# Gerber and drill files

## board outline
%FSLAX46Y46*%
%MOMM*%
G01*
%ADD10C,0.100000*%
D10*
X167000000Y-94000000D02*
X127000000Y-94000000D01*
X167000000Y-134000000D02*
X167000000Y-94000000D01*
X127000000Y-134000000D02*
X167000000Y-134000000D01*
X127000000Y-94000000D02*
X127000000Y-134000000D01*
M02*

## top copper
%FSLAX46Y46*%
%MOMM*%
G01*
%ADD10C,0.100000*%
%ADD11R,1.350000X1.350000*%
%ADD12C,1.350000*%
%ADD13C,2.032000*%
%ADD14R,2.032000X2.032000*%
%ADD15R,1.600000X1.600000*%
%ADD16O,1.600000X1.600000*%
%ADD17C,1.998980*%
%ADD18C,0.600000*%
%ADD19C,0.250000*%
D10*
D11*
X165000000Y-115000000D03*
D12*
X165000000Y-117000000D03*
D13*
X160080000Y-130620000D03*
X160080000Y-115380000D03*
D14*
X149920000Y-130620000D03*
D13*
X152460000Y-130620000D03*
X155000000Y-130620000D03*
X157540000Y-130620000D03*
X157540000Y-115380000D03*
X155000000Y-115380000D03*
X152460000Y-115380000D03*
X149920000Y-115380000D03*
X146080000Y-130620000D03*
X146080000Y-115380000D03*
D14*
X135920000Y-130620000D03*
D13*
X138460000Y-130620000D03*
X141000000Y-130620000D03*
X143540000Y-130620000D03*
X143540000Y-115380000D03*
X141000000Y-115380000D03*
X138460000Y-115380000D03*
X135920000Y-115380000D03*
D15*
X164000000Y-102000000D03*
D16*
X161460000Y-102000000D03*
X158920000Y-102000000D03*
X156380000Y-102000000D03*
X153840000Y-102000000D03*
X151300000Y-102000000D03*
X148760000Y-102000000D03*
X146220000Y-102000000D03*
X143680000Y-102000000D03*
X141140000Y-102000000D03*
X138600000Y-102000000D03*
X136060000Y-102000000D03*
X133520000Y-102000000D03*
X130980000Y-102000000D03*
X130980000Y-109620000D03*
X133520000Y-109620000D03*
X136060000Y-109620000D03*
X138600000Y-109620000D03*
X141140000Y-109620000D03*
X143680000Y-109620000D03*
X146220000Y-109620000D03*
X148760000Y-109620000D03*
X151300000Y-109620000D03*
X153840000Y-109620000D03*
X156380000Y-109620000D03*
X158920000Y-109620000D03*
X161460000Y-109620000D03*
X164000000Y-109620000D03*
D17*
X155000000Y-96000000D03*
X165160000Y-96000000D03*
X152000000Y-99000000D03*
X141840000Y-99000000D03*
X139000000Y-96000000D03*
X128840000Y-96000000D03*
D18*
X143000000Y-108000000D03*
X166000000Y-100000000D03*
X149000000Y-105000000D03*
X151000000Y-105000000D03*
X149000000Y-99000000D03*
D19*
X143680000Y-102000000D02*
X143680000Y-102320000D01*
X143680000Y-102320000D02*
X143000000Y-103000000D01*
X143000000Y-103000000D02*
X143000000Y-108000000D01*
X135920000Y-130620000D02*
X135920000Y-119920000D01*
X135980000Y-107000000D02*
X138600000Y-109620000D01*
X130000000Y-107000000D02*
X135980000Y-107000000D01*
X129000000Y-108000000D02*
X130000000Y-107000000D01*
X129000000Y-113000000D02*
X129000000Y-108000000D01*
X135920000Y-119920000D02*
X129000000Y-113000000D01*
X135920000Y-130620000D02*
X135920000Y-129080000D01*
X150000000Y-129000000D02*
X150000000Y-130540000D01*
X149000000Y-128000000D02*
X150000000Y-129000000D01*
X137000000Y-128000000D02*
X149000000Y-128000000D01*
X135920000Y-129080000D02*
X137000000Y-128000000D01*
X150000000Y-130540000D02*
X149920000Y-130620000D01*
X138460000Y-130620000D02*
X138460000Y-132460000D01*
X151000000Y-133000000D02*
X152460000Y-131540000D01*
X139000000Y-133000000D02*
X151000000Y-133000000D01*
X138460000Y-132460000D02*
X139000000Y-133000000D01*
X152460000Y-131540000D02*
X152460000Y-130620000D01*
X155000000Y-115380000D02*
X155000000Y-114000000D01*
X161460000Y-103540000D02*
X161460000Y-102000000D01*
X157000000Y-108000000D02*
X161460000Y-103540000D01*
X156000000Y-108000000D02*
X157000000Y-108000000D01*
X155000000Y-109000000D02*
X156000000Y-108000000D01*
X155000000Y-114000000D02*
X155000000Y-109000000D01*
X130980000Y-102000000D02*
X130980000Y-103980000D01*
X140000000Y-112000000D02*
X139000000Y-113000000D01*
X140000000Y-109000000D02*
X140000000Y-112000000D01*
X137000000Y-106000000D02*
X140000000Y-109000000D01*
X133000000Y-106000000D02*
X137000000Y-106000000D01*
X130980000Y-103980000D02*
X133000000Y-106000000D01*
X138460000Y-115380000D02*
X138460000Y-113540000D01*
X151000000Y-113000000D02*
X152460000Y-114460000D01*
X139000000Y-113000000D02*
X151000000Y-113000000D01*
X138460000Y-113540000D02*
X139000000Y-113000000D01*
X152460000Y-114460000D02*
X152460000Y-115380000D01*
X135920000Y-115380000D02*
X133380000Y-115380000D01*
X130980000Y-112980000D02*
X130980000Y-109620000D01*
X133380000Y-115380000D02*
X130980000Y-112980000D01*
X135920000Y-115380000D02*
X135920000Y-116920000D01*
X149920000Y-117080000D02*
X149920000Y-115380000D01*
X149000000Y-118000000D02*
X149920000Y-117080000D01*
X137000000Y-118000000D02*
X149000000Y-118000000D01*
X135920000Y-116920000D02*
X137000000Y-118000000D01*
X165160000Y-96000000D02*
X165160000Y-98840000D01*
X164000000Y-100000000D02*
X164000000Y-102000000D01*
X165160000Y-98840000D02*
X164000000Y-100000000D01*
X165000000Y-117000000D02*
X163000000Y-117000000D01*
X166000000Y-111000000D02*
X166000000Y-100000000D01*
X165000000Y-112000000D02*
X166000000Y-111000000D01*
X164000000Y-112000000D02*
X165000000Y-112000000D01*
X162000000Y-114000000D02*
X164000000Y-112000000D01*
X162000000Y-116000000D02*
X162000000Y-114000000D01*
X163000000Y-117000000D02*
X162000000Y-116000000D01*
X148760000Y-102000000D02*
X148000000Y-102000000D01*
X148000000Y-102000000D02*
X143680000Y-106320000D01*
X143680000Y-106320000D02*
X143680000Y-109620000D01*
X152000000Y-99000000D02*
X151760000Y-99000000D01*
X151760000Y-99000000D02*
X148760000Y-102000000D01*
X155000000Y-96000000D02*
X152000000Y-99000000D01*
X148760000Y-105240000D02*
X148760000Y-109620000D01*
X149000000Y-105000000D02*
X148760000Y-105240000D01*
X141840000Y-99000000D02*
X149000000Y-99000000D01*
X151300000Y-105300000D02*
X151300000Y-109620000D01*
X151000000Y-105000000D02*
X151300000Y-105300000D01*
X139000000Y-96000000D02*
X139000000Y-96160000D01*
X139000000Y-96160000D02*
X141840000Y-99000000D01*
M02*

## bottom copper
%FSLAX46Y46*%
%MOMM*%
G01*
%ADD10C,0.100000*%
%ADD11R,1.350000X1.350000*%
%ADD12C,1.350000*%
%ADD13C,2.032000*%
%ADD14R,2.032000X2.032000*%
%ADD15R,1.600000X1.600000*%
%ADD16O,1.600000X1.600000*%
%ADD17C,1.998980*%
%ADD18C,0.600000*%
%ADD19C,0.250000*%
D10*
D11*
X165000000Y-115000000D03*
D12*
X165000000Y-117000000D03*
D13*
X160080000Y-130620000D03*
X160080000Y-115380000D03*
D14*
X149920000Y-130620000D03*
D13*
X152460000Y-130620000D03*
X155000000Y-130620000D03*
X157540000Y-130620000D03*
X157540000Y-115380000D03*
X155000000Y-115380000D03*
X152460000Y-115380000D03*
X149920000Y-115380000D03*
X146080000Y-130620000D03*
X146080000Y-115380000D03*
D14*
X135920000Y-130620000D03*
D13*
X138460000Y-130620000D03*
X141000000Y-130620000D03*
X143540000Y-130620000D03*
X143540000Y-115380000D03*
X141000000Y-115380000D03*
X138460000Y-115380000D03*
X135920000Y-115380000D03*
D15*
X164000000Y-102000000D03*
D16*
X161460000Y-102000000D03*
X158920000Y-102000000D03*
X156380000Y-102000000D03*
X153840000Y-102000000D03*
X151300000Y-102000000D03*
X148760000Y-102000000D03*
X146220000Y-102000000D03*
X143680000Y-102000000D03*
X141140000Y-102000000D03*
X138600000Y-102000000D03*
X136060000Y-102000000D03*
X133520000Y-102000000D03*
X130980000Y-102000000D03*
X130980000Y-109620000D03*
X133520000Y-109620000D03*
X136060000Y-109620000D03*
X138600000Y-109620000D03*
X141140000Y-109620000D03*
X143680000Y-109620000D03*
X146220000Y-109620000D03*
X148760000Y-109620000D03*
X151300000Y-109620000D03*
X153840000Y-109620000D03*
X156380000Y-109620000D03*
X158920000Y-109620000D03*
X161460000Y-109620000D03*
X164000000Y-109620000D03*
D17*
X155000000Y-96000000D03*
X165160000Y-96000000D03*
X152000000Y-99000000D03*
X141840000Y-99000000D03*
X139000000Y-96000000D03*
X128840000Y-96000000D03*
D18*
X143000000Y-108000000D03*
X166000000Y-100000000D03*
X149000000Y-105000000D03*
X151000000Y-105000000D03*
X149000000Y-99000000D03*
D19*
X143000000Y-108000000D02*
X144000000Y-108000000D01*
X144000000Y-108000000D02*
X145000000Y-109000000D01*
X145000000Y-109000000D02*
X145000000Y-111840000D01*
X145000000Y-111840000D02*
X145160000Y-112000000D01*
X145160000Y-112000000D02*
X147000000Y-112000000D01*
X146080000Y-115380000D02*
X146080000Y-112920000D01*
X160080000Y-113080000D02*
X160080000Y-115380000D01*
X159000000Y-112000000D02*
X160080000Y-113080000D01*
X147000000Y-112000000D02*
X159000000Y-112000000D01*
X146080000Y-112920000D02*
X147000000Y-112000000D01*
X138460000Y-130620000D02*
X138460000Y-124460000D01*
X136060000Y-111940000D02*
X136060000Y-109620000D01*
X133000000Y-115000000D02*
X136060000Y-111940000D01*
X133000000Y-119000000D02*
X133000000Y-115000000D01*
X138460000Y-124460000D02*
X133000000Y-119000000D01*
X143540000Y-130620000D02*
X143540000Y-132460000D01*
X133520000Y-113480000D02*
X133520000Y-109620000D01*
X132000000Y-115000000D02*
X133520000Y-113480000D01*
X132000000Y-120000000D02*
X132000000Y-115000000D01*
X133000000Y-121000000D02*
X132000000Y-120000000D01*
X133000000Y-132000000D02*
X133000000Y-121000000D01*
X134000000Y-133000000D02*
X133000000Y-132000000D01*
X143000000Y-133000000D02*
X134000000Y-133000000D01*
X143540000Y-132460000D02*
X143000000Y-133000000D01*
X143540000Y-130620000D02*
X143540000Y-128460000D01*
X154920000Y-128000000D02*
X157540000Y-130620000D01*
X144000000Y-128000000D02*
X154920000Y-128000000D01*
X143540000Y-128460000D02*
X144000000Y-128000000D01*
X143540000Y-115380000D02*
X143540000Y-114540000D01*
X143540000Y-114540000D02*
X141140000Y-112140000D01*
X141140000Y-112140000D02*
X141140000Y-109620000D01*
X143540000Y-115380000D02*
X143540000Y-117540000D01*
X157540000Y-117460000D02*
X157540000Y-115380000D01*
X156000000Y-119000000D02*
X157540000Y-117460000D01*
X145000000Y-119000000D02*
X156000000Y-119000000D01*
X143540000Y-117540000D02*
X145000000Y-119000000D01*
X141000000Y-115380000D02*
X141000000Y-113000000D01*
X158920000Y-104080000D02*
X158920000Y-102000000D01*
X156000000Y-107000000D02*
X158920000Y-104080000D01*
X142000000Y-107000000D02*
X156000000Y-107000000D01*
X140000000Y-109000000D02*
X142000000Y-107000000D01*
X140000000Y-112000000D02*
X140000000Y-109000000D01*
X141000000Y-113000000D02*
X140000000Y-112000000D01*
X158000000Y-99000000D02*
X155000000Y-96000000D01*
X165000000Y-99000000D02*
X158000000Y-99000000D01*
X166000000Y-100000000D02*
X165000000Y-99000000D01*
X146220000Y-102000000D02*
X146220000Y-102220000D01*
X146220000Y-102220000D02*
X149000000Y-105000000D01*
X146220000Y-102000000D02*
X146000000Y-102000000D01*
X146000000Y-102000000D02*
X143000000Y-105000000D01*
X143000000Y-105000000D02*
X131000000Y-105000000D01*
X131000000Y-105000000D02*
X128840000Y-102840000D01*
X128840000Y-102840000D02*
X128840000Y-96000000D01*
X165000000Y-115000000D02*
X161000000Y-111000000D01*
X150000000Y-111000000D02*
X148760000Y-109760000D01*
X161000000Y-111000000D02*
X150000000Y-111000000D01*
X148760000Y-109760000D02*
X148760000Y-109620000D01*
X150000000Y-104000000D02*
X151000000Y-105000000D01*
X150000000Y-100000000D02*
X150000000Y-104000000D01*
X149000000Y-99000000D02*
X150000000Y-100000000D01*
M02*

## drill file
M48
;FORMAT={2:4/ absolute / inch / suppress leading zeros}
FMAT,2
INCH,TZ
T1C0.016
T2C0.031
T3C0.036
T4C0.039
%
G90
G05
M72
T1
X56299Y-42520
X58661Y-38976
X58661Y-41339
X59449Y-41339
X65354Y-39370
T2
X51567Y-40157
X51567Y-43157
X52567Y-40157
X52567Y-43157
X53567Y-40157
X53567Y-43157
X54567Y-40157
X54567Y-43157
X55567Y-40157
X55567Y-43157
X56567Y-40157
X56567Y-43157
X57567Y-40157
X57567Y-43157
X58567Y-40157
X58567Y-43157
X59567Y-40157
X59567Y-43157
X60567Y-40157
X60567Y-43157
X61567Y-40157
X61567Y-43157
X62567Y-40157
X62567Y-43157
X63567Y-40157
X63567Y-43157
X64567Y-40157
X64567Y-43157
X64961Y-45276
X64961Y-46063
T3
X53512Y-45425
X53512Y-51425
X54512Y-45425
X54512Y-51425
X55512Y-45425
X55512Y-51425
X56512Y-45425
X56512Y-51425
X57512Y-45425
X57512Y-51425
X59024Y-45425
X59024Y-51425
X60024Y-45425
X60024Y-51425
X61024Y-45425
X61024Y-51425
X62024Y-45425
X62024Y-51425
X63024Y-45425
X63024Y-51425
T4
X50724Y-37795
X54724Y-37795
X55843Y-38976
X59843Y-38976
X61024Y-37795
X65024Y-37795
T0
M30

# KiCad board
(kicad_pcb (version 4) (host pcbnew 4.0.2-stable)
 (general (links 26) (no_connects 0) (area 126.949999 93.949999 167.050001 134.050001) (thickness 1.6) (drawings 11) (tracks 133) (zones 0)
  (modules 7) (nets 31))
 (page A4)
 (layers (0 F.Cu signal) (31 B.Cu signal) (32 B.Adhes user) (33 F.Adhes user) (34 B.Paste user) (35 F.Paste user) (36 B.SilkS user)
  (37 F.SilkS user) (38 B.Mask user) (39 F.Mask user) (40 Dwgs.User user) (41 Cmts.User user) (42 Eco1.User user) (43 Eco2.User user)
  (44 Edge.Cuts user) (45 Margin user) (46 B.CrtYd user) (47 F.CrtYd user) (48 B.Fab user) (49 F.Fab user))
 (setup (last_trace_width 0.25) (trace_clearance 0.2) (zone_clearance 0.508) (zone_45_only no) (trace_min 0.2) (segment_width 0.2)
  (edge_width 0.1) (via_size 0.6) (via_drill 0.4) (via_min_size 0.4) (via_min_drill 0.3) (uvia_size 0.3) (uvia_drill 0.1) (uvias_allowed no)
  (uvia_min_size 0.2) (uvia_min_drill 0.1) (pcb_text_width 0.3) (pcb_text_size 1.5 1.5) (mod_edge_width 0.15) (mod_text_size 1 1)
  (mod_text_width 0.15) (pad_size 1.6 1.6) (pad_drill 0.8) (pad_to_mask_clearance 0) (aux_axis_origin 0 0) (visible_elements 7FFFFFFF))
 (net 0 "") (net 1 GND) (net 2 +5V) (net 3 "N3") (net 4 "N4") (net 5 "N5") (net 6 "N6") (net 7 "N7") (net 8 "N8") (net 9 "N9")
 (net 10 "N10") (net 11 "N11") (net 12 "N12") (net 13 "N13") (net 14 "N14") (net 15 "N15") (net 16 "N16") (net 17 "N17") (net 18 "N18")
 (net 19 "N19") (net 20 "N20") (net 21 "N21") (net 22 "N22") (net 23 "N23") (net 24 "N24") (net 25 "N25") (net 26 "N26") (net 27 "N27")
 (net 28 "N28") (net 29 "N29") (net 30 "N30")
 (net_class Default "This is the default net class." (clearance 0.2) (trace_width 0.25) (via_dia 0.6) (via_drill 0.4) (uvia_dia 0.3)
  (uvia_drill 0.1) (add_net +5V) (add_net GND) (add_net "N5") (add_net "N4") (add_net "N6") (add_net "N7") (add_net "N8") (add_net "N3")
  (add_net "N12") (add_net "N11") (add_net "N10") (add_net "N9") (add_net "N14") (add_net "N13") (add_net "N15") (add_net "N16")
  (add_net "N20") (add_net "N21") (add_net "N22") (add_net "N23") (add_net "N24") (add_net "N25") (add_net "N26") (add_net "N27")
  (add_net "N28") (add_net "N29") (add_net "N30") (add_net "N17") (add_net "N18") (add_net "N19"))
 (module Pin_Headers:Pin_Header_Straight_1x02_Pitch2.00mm (layer F.Cu) (at 165 115)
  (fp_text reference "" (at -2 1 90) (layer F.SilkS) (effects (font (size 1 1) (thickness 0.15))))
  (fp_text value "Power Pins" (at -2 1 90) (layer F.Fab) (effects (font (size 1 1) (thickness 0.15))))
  (pad 1 thru_hole rect (at 0 0) (size 1.35 1.35) (drill 0.8) (layers *.Cu *.Mask) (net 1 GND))
  (pad 2 thru_hole circle (at 0 2) (size 1.35 1.35) (drill 0.8) (layers *.Cu *.Mask) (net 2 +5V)))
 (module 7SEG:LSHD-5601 (layer F.Cu) (at 155 123)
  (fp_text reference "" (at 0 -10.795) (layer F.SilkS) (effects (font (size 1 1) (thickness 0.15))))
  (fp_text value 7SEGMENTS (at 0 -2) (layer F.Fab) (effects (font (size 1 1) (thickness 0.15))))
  (pad 5 thru_hole circle (at 5.08 7.62) (size 2.032 2.032) (drill 0.9144) (layers *.Cu *.Mask F.SilkS) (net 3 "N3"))
  (pad 10 thru_hole circle (at 5.08 -7.62) (size 2.032 2.032) (drill 0.9144) (layers *.Cu *.Mask F.SilkS) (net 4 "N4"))
  (pad 1 thru_hole rect (at -5.08 7.62) (size 2.032 2.032) (drill 0.9144) (layers *.Cu *.Mask F.SilkS) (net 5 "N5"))
  (pad 2 thru_hole circle (at -2.54 7.62) (size 2.032 2.032) (drill 0.9144) (layers *.Cu *.Mask F.SilkS) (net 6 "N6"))
  (pad 3 thru_hole circle (at 0 7.62) (size 2.032 2.032) (drill 0.9144) (layers *.Cu *.Mask F.SilkS) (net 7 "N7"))
  (pad 4 thru_hole circle (at 2.54 7.62) (size 2.032 2.032) (drill 0.9144) (layers *.Cu *.Mask F.SilkS) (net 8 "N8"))
  (pad 9 thru_hole circle (at 2.54 -7.62) (size 2.032 2.032) (drill 0.9144) (layers *.Cu *.Mask F.SilkS) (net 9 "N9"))
  (pad 8 thru_hole circle (at 0 -7.62) (size 2.032 2.032) (drill 0.9144) (layers *.Cu *.Mask F.SilkS) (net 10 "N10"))
  (pad 7 thru_hole circle (at -2.54 -7.62) (size 2.032 2.032) (drill 0.9144) (layers *.Cu *.Mask F.SilkS) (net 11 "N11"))
  (pad 6 thru_hole circle (at -5.08 -7.62) (size 2.032 2.032) (drill 0.9144) (layers *.Cu *.Mask F.SilkS) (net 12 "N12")))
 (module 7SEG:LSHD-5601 (layer F.Cu) (at 141 123)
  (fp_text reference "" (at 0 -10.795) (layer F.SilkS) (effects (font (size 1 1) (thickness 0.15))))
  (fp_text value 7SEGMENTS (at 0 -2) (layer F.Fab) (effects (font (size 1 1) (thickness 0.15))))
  (pad 5 thru_hole circle (at 5.08 7.62) (size 2.032 2.032) (drill 0.9144) (layers *.Cu *.Mask F.SilkS) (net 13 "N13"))
  (pad 10 thru_hole circle (at 5.08 -7.62) (size 2.032 2.032) (drill 0.9144) (layers *.Cu *.Mask F.SilkS) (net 4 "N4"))
  (pad 1 thru_hole rect (at -5.08 7.62) (size 2.032 2.032) (drill 0.9144) (layers *.Cu *.Mask F.SilkS) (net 5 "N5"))
  (pad 2 thru_hole circle (at -2.54 7.62) (size 2.032 2.032) (drill 0.9144) (layers *.Cu *.Mask F.SilkS) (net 6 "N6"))
  (pad 3 thru_hole circle (at 0 7.62) (size 2.032 2.032) (drill 0.9144) (layers *.Cu *.Mask F.SilkS) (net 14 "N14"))
  (pad 4 thru_hole circle (at 2.54 7.62) (size 2.032 2.032) (drill 0.9144) (layers *.Cu *.Mask F.SilkS) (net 8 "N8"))
  (pad 9 thru_hole circle (at 2.54 -7.62) (size 2.032 2.032) (drill 0.9144) (layers *.Cu *.Mask F.SilkS) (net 9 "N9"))
  (pad 8 thru_hole circle (at 0 -7.62) (size 2.032 2.032) (drill 0.9144) (layers *.Cu *.Mask F.SilkS) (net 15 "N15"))
  (pad 7 thru_hole circle (at -2.54 -7.62) (size 2.032 2.032) (drill 0.9144) (layers *.Cu *.Mask F.SilkS) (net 11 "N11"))
  (pad 6 thru_hole circle (at -5.08 -7.62) (size 2.032 2.032) (drill 0.9144) (layers *.Cu *.Mask F.SilkS) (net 12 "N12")))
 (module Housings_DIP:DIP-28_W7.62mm (layer F.Cu) (at 164 102 270)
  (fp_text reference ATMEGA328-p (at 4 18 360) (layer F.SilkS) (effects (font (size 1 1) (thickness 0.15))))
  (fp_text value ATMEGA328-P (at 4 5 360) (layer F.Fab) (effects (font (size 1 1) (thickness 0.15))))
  (pad 1 thru_hole rect (at 0 0 270) (size 1.6 1.6) (drill 0.8) (layers *.Cu *.Mask F.SilkS) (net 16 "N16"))
  (pad 2 thru_hole oval (at 0 2.54 270) (size 1.6 1.6) (drill 0.8) (layers *.Cu *.Mask F.SilkS) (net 10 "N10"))
  (pad 3 thru_hole oval (at 0 5.08 270) (size 1.6 1.6) (drill 0.8) (layers *.Cu *.Mask F.SilkS) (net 15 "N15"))
  (pad 4 thru_hole oval (at 0 7.62 270) (size 1.6 1.6) (drill 0.8) (layers *.Cu *.Mask F.SilkS) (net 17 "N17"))
  (pad 5 thru_hole oval (at 0 10.16 270) (size 1.6 1.6) (drill 0.8) (layers *.Cu *.Mask F.SilkS) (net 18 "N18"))
  (pad 6 thru_hole oval (at 0 12.7 270) (size 1.6 1.6) (drill 0.8) (layers *.Cu *.Mask F.SilkS) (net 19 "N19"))
  (pad 7 thru_hole oval (at 0 15.24 270) (size 1.6 1.6) (drill 0.8) (layers *.Cu *.Mask F.SilkS) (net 2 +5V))
  (pad 8 thru_hole oval (at 0 17.78 270) (size 1.6 1.6) (drill 0.8) (layers *.Cu *.Mask F.SilkS) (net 1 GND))
  (pad 9 thru_hole oval (at 0 20.32 270) (size 1.6 1.6) (drill 0.8) (layers *.Cu *.Mask F.SilkS) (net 4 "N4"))
  (pad 10 thru_hole oval (at 0 22.86 270) (size 1.6 1.6) (drill 0.8) (layers *.Cu *.Mask F.SilkS) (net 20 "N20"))
  (pad 11 thru_hole oval (at 0 25.4 270) (size 1.6 1.6) (drill 0.8) (layers *.Cu *.Mask F.SilkS) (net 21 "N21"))
  (pad 12 thru_hole oval (at 0 27.94 270) (size 1.6 1.6) (drill 0.8) (layers *.Cu *.Mask F.SilkS) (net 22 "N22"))
  (pad 13 thru_hole oval (at 0 30.48 270) (size 1.6 1.6) (drill 0.8) (layers *.Cu *.Mask F.SilkS) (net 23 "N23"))
  (pad 14 thru_hole oval (at 0 33.02 270) (size 1.6 1.6) (drill 0.8) (layers *.Cu *.Mask F.SilkS) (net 11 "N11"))
  (pad 15 thru_hole oval (at 7.62 33.02 270) (size 1.6 1.6) (drill 0.8) (layers *.Cu *.Mask F.SilkS) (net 12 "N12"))
  (pad 16 thru_hole oval (at 7.62 30.48 270) (size 1.6 1.6) (drill 0.8) (layers *.Cu *.Mask F.SilkS) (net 8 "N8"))
  (pad 17 thru_hole oval (at 7.62 27.94 270) (size 1.6 1.6) (drill 0.8) (layers *.Cu *.Mask F.SilkS) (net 6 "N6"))
  (pad 18 thru_hole oval (at 7.62 25.4 270) (size 1.6 1.6) (drill 0.8) (layers *.Cu *.Mask F.SilkS) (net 5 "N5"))
  (pad 19 thru_hole oval (at 7.62 22.86 270) (size 1.6 1.6) (drill 0.8) (layers *.Cu *.Mask F.SilkS) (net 9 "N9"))
  (pad 20 thru_hole oval (at 7.62 20.32 270) (size 1.6 1.6) (drill 0.8) (layers *.Cu *.Mask F.SilkS) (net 2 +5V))
  (pad 21 thru_hole oval (at 7.62 17.78 270) (size 1.6 1.6) (drill 0.8) (layers *.Cu *.Mask F.SilkS) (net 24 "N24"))
  (pad 22 thru_hole oval (at 7.62 15.24 270) (size 1.6 1.6) (drill 0.8) (layers *.Cu *.Mask F.SilkS) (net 1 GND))
  (pad 23 thru_hole oval (at 7.62 12.7 270) (size 1.6 1.6) (drill 0.8) (layers *.Cu *.Mask F.SilkS) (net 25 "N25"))
  (pad 24 thru_hole oval (at 7.62 10.16 270) (size 1.6 1.6) (drill 0.8) (layers *.Cu *.Mask F.SilkS) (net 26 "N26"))
  (pad 25 thru_hole oval (at 7.62 7.62 270) (size 1.6 1.6) (drill 0.8) (layers *.Cu *.Mask F.SilkS) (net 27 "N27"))
  (pad 26 thru_hole oval (at 7.62 5.08 270) (size 1.6 1.6) (drill 0.8) (layers *.Cu *.Mask F.SilkS) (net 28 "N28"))
  (pad 27 thru_hole oval (at 7.62 2.54 270) (size 1.6 1.6) (drill 0.8) (layers *.Cu *.Mask F.SilkS) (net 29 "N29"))
  (pad 28 thru_hole oval (at 7.62 0 270) (size 1.6 1.6) (drill 0.8) (layers *.Cu *.Mask F.SilkS) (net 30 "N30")))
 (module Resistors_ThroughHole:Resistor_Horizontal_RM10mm (layer F.Cu) (at 155 96)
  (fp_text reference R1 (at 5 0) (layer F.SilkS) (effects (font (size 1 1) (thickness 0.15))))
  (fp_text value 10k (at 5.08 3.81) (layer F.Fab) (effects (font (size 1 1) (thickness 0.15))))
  (pad 1 thru_hole circle (at 0 0) (size 1.99898 1.99898) (drill 1.00076) (layers *.Cu *.SilkS *.Mask) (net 2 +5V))
  (pad 2 thru_hole circle (at 10.16 0) (size 1.99898 1.99898) (drill 1.00076) (layers *.Cu *.SilkS *.Mask) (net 16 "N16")))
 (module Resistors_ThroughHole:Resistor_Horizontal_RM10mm (layer F.Cu) (at 152 99 180)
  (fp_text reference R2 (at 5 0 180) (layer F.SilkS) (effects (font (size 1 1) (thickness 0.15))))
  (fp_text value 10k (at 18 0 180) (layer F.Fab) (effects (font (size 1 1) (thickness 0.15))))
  (pad 1 thru_hole circle (at 0 0 180) (size 1.99898 1.99898) (drill 1.00076) (layers *.Cu *.SilkS *.Mask) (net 2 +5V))
  (pad 2 thru_hole circle (at 10.16 0 180) (size 1.99898 1.99898) (drill 1.00076) (layers *.Cu *.SilkS *.Mask) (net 25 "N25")))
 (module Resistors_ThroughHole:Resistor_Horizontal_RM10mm (layer F.Cu) (at 139 96 180)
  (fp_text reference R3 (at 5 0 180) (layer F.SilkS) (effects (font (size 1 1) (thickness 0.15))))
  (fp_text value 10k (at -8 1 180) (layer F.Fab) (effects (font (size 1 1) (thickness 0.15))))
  (pad 1 thru_hole circle (at 0 0 180) (size 1.99898 1.99898) (drill 1.00076) (layers *.Cu *.SilkS *.Mask) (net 25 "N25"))
  (pad 2 thru_hole circle (at 10.16 0 180) (size 1.99898 1.99898) (drill 1.00076) (layers *.Cu *.SilkS *.Mask) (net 1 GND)))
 (gr_line (start 167 94) (end 127 94) (angle 90) (layer Edge.Cuts) (width 0.1))
 (gr_line (start 167 134) (end 167 94) (angle 90) (layer Edge.Cuts) (width 0.1))
 (gr_line (start 127 134) (end 167 134) (angle 90) (layer Edge.Cuts) (width 0.1))
 (gr_line (start 127 94) (end 127 134) (angle 90) (layer Edge.Cuts) (width 0.1))
 (segment (start 143.68 102) (end 143.68 102.32) (width 0.25) (layer F.Cu) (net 4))
 (segment (start 143.68 102.32) (end 143 103) (width 0.25) (layer F.Cu) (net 4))
 (segment (start 143 103) (end 143 108) (width 0.25) (layer F.Cu) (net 4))
 (via (at 143 108) (size 0.6) (drill 0.4) (layers F.Cu B.Cu) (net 4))
 (segment (start 143 108) (end 144 108) (width 0.25) (layer B.Cu) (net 4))
 (segment (start 144 108) (end 145 109) (width 0.25) (layer B.Cu) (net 4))
 (segment (start 145 109) (end 145 111.84) (width 0.25) (layer B.Cu) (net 4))
 (segment (start 145 111.84) (end 145.16 112) (width 0.25) (layer B.Cu) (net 4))
 (segment (start 145.16 112) (end 147 112) (width 0.25) (layer B.Cu) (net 4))
 (segment (start 146.08 115.38) (end 146.08 112.92) (width 0.25) (layer B.Cu) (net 4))
 (segment (start 160.08 113.08) (end 160.08 115.38) (width 0.25) (layer B.Cu) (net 4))
 (segment (start 159 112) (end 160.08 113.08) (width 0.25) (layer B.Cu) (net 4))
 (segment (start 147 112) (end 159 112) (width 0.25) (layer B.Cu) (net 4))
 (segment (start 146.08 112.92) (end 147 112) (width 0.25) (layer B.Cu) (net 4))
 (segment (start 135.92 130.62) (end 135.92 119.92) (width 0.25) (layer F.Cu) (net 5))
 (segment (start 135.98 107) (end 138.6 109.62) (width 0.25) (layer F.Cu) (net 5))
 (segment (start 130 107) (end 135.98 107) (width 0.25) (layer F.Cu) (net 5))
 (segment (start 129 108) (end 130 107) (width 0.25) (layer F.Cu) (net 5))
 (segment (start 129 113) (end 129 108) (width 0.25) (layer F.Cu) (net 5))
 (segment (start 135.92 119.92) (end 129 113) (width 0.25) (layer F.Cu) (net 5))
 (segment (start 135.92 130.62) (end 135.92 129.08) (width 0.25) (layer F.Cu) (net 5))
 (segment (start 150 129) (end 150 130.54) (width 0.25) (layer F.Cu) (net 5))
 (segment (start 149 128) (end 150 129) (width 0.25) (layer F.Cu) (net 5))
 (segment (start 137 128) (end 149 128) (width 0.25) (layer F.Cu) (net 5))
 (segment (start 135.92 129.08) (end 137 128) (width 0.25) (layer F.Cu) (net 5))
 (segment (start 150 130.54) (end 149.92 130.62) (width 0.25) (layer F.Cu) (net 5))
 (segment (start 138.46 130.62) (end 138.46 124.46) (width 0.25) (layer B.Cu) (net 6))
 (segment (start 136.06 111.94) (end 136.06 109.62) (width 0.25) (layer B.Cu) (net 6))
 (segment (start 133 115) (end 136.06 111.94) (width 0.25) (layer B.Cu) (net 6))
 (segment (start 133 119) (end 133 115) (width 0.25) (layer B.Cu) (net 6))
 (segment (start 138.46 124.46) (end 133 119) (width 0.25) (layer B.Cu) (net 6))
 (segment (start 138.46 130.62) (end 138.46 132.46) (width 0.25) (layer F.Cu) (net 6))
 (segment (start 151 133) (end 152.46 131.54) (width 0.25) (layer F.Cu) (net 6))
 (segment (start 139 133) (end 151 133) (width 0.25) (layer F.Cu) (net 6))
 (segment (start 138.46 132.46) (end 139 133) (width 0.25) (layer F.Cu) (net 6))
 (segment (start 152.46 131.54) (end 152.46 130.62) (width 0.25) (layer F.Cu) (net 6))
 (segment (start 143.54 130.62) (end 143.54 132.46) (width 0.25) (layer B.Cu) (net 8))
 (segment (start 133.52 113.48) (end 133.52 109.62) (width 0.25) (layer B.Cu) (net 8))
 (segment (start 132 115) (end 133.52 113.48) (width 0.25) (layer B.Cu) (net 8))
 (segment (start 132 120) (end 132 115) (width 0.25) (layer B.Cu) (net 8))
 (segment (start 133 121) (end 132 120) (width 0.25) (layer B.Cu) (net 8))
 (segment (start 133 132) (end 133 121) (width 0.25) (layer B.Cu) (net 8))
 (segment (start 134 133) (end 133 132) (width 0.25) (layer B.Cu) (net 8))
 (segment (start 143 133) (end 134 133) (width 0.25) (layer B.Cu) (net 8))
 (segment (start 143.54 132.46) (end 143 133) (width 0.25) (layer B.Cu) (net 8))
 (segment (start 143.54 130.62) (end 143.54 128.46) (width 0.25) (layer B.Cu) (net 8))
 (segment (start 154.92 128) (end 157.54 130.62) (width 0.25) (layer B.Cu) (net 8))
 (segment (start 144 128) (end 154.92 128) (width 0.25) (layer B.Cu) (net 8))
 (segment (start 143.54 128.46) (end 144 128) (width 0.25) (layer B.Cu) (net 8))
 (segment (start 143.54 115.38) (end 143.54 114.54) (width 0.25) (layer B.Cu) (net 9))
 (segment (start 143.54 114.54) (end 141.14 112.14) (width 0.25) (layer B.Cu) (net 9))
 (segment (start 141.14 112.14) (end 141.14 109.62) (width 0.25) (layer B.Cu) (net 9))
 (segment (start 143.54 115.38) (end 143.54 117.54) (width 0.25) (layer B.Cu) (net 9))
 (segment (start 157.54 117.46) (end 157.54 115.38) (width 0.25) (layer B.Cu) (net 9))
 (segment (start 156 119) (end 157.54 117.46) (width 0.25) (layer B.Cu) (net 9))
 (segment (start 145 119) (end 156 119) (width 0.25) (layer B.Cu) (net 9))
 (segment (start 143.54 117.54) (end 145 119) (width 0.25) (layer B.Cu) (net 9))
 (segment (start 155 115.38) (end 155 114) (width 0.25) (layer F.Cu) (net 10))
 (segment (start 161.46 103.54) (end 161.46 102) (width 0.25) (layer F.Cu) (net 10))
 (segment (start 157 108) (end 161.46 103.54) (width 0.25) (layer F.Cu) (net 10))
 (segment (start 156 108) (end 157 108) (width 0.25) (layer F.Cu) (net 10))
 (segment (start 155 109) (end 156 108) (width 0.25) (layer F.Cu) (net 10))
 (segment (start 155 114) (end 155 109) (width 0.25) (layer F.Cu) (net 10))
 (segment (start 130.98 102) (end 130.98 103.98) (width 0.25) (layer F.Cu) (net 11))
 (segment (start 140 112) (end 139 113) (width 0.25) (layer F.Cu) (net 11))
 (segment (start 140 109) (end 140 112) (width 0.25) (layer F.Cu) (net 11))
 (segment (start 137 106) (end 140 109) (width 0.25) (layer F.Cu) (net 11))
 (segment (start 133 106) (end 137 106) (width 0.25) (layer F.Cu) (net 11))
 (segment (start 130.98 103.98) (end 133 106) (width 0.25) (layer F.Cu) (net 11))
 (segment (start 138.46 115.38) (end 138.46 113.54) (width 0.25) (layer F.Cu) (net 11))
 (segment (start 151 113) (end 152.46 114.46) (width 0.25) (layer F.Cu) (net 11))
 (segment (start 139 113) (end 151 113) (width 0.25) (layer F.Cu) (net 11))
 (segment (start 138.46 113.54) (end 139 113) (width 0.25) (layer F.Cu) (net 11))
 (segment (start 152.46 114.46) (end 152.46 115.38) (width 0.25) (layer F.Cu) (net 11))
 (segment (start 135.92 115.38) (end 133.38 115.38) (width 0.25) (layer F.Cu) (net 12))
 (segment (start 130.98 112.98) (end 130.98 109.62) (width 0.25) (layer F.Cu) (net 12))
 (segment (start 133.38 115.38) (end 130.98 112.98) (width 0.25) (layer F.Cu) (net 12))
 (segment (start 135.92 115.38) (end 135.92 116.92) (width 0.25) (layer F.Cu) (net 12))
 (segment (start 149.92 117.08) (end 149.92 115.38) (width 0.25) (layer F.Cu) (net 12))
 (segment (start 149 118) (end 149.92 117.08) (width 0.25) (layer F.Cu) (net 12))
 (segment (start 137 118) (end 149 118) (width 0.25) (layer F.Cu) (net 12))
 (segment (start 135.92 116.92) (end 137 118) (width 0.25) (layer F.Cu) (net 12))
 (segment (start 141 115.38) (end 141 113) (width 0.25) (layer B.Cu) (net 15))
 (segment (start 158.92 104.08) (end 158.92 102) (width 0.25) (layer B.Cu) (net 15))
 (segment (start 156 107) (end 158.92 104.08) (width 0.25) (layer B.Cu) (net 15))
 (segment (start 142 107) (end 156 107) (width 0.25) (layer B.Cu) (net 15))
 (segment (start 140 109) (end 142 107) (width 0.25) (layer B.Cu) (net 15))
 (segment (start 140 112) (end 140 109) (width 0.25) (layer B.Cu) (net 15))
 (segment (start 141 113) (end 140 112) (width 0.25) (layer B.Cu) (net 15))
 (segment (start 165.16 96) (end 165.16 98.84) (width 0.25) (layer F.Cu) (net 16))
 (segment (start 164 100) (end 164 102) (width 0.25) (layer F.Cu) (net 16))
 (segment (start 165.16 98.84) (end 164 100) (width 0.25) (layer F.Cu) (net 16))
 (segment (start 165 117) (end 163 117) (width 0.25) (layer F.Cu) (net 2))
 (segment (start 158 99) (end 155 96) (width 0.25) (layer B.Cu) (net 2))
 (segment (start 165 99) (end 158 99) (width 0.25) (layer B.Cu) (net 2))
 (segment (start 166 100) (end 165 99) (width 0.25) (layer B.Cu) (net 2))
 (via (at 166 100) (size 0.6) (drill 0.4) (layers F.Cu B.Cu) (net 2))
 (segment (start 166 111) (end 166 100) (width 0.25) (layer F.Cu) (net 2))
 (segment (start 165 112) (end 166 111) (width 0.25) (layer F.Cu) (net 2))
 (segment (start 164 112) (end 165 112) (width 0.25) (layer F.Cu) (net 2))
 (segment (start 162 114) (end 164 112) (width 0.25) (layer F.Cu) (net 2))
 (segment (start 162 116) (end 162 114) (width 0.25) (layer F.Cu) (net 2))
 (segment (start 163 117) (end 162 116) (width 0.25) (layer F.Cu) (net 2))
 (segment (start 148.76 102) (end 148 102) (width 0.25) (layer F.Cu) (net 2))
 (segment (start 148 102) (end 143.68 106.32) (width 0.25) (layer F.Cu) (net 2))
 (segment (start 143.68 106.32) (end 143.68 109.62) (width 0.25) (layer F.Cu) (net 2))
 (segment (start 152 99) (end 151.76 99) (width 0.25) (layer F.Cu) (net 2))
 (segment (start 151.76 99) (end 148.76 102) (width 0.25) (layer F.Cu) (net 2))
 (segment (start 155 96) (end 152 99) (width 0.25) (layer F.Cu) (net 2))
 (segment (start 146.22 102) (end 146.22 102.22) (width 0.25) (layer B.Cu) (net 1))
 (segment (start 146.22 102.22) (end 149 105) (width 0.25) (layer B.Cu) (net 1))
 (segment (start 148.76 105.24) (end 148.76 109.62) (width 0.25) (layer F.Cu) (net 1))
 (segment (start 149 105) (end 148.76 105.24) (width 0.25) (layer F.Cu) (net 1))
 (via (at 149 105) (size 0.6) (drill 0.4) (layers F.Cu B.Cu) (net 1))
 (segment (start 146.22 102) (end 146 102) (width 0.25) (layer B.Cu) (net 1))
 (segment (start 146 102) (end 143 105) (width 0.25) (layer B.Cu) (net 1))
 (segment (start 143 105) (end 131 105) (width 0.25) (layer B.Cu) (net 1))
 (segment (start 131 105) (end 128.84 102.84) (width 0.25) (layer B.Cu) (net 1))
 (segment (start 128.84 102.84) (end 128.84 96) (width 0.25) (layer B.Cu) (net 1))
 (segment (start 165 115) (end 161 111) (width 0.25) (layer B.Cu) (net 1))
 (segment (start 150 111) (end 148.76 109.76) (width 0.25) (layer B.Cu) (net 1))
 (segment (start 161 111) (end 150 111) (width 0.25) (layer B.Cu) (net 1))
 (segment (start 148.76 109.76) (end 148.76 109.62) (width 0.25) (layer B.Cu) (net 1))
 (segment (start 141.84 99) (end 149 99) (width 0.25) (layer F.Cu) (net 25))
 (segment (start 151.3 105.3) (end 151.3 109.62) (width 0.25) (layer F.Cu) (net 25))
 (segment (start 151 105) (end 151.3 105.3) (width 0.25) (layer F.Cu) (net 25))
 (via (at 151 105) (size 0.6) (drill 0.4) (layers F.Cu B.Cu) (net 25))
 (segment (start 150 104) (end 151 105) (width 0.25) (layer B.Cu) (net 25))
 (segment (start 150 100) (end 150 104) (width 0.25) (layer B.Cu) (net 25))
 (segment (start 149 99) (end 150 100) (width 0.25) (layer B.Cu) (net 25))
 (via (at 149 99) (size 0.6) (drill 0.4) (layers F.Cu B.Cu) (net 25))
 (segment (start 139 96) (end 139 96.16) (width 0.25) (layer F.Cu) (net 25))
 (segment (start 139 96.16) (end 141.84 99) (width 0.25) (layer F.Cu) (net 25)))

